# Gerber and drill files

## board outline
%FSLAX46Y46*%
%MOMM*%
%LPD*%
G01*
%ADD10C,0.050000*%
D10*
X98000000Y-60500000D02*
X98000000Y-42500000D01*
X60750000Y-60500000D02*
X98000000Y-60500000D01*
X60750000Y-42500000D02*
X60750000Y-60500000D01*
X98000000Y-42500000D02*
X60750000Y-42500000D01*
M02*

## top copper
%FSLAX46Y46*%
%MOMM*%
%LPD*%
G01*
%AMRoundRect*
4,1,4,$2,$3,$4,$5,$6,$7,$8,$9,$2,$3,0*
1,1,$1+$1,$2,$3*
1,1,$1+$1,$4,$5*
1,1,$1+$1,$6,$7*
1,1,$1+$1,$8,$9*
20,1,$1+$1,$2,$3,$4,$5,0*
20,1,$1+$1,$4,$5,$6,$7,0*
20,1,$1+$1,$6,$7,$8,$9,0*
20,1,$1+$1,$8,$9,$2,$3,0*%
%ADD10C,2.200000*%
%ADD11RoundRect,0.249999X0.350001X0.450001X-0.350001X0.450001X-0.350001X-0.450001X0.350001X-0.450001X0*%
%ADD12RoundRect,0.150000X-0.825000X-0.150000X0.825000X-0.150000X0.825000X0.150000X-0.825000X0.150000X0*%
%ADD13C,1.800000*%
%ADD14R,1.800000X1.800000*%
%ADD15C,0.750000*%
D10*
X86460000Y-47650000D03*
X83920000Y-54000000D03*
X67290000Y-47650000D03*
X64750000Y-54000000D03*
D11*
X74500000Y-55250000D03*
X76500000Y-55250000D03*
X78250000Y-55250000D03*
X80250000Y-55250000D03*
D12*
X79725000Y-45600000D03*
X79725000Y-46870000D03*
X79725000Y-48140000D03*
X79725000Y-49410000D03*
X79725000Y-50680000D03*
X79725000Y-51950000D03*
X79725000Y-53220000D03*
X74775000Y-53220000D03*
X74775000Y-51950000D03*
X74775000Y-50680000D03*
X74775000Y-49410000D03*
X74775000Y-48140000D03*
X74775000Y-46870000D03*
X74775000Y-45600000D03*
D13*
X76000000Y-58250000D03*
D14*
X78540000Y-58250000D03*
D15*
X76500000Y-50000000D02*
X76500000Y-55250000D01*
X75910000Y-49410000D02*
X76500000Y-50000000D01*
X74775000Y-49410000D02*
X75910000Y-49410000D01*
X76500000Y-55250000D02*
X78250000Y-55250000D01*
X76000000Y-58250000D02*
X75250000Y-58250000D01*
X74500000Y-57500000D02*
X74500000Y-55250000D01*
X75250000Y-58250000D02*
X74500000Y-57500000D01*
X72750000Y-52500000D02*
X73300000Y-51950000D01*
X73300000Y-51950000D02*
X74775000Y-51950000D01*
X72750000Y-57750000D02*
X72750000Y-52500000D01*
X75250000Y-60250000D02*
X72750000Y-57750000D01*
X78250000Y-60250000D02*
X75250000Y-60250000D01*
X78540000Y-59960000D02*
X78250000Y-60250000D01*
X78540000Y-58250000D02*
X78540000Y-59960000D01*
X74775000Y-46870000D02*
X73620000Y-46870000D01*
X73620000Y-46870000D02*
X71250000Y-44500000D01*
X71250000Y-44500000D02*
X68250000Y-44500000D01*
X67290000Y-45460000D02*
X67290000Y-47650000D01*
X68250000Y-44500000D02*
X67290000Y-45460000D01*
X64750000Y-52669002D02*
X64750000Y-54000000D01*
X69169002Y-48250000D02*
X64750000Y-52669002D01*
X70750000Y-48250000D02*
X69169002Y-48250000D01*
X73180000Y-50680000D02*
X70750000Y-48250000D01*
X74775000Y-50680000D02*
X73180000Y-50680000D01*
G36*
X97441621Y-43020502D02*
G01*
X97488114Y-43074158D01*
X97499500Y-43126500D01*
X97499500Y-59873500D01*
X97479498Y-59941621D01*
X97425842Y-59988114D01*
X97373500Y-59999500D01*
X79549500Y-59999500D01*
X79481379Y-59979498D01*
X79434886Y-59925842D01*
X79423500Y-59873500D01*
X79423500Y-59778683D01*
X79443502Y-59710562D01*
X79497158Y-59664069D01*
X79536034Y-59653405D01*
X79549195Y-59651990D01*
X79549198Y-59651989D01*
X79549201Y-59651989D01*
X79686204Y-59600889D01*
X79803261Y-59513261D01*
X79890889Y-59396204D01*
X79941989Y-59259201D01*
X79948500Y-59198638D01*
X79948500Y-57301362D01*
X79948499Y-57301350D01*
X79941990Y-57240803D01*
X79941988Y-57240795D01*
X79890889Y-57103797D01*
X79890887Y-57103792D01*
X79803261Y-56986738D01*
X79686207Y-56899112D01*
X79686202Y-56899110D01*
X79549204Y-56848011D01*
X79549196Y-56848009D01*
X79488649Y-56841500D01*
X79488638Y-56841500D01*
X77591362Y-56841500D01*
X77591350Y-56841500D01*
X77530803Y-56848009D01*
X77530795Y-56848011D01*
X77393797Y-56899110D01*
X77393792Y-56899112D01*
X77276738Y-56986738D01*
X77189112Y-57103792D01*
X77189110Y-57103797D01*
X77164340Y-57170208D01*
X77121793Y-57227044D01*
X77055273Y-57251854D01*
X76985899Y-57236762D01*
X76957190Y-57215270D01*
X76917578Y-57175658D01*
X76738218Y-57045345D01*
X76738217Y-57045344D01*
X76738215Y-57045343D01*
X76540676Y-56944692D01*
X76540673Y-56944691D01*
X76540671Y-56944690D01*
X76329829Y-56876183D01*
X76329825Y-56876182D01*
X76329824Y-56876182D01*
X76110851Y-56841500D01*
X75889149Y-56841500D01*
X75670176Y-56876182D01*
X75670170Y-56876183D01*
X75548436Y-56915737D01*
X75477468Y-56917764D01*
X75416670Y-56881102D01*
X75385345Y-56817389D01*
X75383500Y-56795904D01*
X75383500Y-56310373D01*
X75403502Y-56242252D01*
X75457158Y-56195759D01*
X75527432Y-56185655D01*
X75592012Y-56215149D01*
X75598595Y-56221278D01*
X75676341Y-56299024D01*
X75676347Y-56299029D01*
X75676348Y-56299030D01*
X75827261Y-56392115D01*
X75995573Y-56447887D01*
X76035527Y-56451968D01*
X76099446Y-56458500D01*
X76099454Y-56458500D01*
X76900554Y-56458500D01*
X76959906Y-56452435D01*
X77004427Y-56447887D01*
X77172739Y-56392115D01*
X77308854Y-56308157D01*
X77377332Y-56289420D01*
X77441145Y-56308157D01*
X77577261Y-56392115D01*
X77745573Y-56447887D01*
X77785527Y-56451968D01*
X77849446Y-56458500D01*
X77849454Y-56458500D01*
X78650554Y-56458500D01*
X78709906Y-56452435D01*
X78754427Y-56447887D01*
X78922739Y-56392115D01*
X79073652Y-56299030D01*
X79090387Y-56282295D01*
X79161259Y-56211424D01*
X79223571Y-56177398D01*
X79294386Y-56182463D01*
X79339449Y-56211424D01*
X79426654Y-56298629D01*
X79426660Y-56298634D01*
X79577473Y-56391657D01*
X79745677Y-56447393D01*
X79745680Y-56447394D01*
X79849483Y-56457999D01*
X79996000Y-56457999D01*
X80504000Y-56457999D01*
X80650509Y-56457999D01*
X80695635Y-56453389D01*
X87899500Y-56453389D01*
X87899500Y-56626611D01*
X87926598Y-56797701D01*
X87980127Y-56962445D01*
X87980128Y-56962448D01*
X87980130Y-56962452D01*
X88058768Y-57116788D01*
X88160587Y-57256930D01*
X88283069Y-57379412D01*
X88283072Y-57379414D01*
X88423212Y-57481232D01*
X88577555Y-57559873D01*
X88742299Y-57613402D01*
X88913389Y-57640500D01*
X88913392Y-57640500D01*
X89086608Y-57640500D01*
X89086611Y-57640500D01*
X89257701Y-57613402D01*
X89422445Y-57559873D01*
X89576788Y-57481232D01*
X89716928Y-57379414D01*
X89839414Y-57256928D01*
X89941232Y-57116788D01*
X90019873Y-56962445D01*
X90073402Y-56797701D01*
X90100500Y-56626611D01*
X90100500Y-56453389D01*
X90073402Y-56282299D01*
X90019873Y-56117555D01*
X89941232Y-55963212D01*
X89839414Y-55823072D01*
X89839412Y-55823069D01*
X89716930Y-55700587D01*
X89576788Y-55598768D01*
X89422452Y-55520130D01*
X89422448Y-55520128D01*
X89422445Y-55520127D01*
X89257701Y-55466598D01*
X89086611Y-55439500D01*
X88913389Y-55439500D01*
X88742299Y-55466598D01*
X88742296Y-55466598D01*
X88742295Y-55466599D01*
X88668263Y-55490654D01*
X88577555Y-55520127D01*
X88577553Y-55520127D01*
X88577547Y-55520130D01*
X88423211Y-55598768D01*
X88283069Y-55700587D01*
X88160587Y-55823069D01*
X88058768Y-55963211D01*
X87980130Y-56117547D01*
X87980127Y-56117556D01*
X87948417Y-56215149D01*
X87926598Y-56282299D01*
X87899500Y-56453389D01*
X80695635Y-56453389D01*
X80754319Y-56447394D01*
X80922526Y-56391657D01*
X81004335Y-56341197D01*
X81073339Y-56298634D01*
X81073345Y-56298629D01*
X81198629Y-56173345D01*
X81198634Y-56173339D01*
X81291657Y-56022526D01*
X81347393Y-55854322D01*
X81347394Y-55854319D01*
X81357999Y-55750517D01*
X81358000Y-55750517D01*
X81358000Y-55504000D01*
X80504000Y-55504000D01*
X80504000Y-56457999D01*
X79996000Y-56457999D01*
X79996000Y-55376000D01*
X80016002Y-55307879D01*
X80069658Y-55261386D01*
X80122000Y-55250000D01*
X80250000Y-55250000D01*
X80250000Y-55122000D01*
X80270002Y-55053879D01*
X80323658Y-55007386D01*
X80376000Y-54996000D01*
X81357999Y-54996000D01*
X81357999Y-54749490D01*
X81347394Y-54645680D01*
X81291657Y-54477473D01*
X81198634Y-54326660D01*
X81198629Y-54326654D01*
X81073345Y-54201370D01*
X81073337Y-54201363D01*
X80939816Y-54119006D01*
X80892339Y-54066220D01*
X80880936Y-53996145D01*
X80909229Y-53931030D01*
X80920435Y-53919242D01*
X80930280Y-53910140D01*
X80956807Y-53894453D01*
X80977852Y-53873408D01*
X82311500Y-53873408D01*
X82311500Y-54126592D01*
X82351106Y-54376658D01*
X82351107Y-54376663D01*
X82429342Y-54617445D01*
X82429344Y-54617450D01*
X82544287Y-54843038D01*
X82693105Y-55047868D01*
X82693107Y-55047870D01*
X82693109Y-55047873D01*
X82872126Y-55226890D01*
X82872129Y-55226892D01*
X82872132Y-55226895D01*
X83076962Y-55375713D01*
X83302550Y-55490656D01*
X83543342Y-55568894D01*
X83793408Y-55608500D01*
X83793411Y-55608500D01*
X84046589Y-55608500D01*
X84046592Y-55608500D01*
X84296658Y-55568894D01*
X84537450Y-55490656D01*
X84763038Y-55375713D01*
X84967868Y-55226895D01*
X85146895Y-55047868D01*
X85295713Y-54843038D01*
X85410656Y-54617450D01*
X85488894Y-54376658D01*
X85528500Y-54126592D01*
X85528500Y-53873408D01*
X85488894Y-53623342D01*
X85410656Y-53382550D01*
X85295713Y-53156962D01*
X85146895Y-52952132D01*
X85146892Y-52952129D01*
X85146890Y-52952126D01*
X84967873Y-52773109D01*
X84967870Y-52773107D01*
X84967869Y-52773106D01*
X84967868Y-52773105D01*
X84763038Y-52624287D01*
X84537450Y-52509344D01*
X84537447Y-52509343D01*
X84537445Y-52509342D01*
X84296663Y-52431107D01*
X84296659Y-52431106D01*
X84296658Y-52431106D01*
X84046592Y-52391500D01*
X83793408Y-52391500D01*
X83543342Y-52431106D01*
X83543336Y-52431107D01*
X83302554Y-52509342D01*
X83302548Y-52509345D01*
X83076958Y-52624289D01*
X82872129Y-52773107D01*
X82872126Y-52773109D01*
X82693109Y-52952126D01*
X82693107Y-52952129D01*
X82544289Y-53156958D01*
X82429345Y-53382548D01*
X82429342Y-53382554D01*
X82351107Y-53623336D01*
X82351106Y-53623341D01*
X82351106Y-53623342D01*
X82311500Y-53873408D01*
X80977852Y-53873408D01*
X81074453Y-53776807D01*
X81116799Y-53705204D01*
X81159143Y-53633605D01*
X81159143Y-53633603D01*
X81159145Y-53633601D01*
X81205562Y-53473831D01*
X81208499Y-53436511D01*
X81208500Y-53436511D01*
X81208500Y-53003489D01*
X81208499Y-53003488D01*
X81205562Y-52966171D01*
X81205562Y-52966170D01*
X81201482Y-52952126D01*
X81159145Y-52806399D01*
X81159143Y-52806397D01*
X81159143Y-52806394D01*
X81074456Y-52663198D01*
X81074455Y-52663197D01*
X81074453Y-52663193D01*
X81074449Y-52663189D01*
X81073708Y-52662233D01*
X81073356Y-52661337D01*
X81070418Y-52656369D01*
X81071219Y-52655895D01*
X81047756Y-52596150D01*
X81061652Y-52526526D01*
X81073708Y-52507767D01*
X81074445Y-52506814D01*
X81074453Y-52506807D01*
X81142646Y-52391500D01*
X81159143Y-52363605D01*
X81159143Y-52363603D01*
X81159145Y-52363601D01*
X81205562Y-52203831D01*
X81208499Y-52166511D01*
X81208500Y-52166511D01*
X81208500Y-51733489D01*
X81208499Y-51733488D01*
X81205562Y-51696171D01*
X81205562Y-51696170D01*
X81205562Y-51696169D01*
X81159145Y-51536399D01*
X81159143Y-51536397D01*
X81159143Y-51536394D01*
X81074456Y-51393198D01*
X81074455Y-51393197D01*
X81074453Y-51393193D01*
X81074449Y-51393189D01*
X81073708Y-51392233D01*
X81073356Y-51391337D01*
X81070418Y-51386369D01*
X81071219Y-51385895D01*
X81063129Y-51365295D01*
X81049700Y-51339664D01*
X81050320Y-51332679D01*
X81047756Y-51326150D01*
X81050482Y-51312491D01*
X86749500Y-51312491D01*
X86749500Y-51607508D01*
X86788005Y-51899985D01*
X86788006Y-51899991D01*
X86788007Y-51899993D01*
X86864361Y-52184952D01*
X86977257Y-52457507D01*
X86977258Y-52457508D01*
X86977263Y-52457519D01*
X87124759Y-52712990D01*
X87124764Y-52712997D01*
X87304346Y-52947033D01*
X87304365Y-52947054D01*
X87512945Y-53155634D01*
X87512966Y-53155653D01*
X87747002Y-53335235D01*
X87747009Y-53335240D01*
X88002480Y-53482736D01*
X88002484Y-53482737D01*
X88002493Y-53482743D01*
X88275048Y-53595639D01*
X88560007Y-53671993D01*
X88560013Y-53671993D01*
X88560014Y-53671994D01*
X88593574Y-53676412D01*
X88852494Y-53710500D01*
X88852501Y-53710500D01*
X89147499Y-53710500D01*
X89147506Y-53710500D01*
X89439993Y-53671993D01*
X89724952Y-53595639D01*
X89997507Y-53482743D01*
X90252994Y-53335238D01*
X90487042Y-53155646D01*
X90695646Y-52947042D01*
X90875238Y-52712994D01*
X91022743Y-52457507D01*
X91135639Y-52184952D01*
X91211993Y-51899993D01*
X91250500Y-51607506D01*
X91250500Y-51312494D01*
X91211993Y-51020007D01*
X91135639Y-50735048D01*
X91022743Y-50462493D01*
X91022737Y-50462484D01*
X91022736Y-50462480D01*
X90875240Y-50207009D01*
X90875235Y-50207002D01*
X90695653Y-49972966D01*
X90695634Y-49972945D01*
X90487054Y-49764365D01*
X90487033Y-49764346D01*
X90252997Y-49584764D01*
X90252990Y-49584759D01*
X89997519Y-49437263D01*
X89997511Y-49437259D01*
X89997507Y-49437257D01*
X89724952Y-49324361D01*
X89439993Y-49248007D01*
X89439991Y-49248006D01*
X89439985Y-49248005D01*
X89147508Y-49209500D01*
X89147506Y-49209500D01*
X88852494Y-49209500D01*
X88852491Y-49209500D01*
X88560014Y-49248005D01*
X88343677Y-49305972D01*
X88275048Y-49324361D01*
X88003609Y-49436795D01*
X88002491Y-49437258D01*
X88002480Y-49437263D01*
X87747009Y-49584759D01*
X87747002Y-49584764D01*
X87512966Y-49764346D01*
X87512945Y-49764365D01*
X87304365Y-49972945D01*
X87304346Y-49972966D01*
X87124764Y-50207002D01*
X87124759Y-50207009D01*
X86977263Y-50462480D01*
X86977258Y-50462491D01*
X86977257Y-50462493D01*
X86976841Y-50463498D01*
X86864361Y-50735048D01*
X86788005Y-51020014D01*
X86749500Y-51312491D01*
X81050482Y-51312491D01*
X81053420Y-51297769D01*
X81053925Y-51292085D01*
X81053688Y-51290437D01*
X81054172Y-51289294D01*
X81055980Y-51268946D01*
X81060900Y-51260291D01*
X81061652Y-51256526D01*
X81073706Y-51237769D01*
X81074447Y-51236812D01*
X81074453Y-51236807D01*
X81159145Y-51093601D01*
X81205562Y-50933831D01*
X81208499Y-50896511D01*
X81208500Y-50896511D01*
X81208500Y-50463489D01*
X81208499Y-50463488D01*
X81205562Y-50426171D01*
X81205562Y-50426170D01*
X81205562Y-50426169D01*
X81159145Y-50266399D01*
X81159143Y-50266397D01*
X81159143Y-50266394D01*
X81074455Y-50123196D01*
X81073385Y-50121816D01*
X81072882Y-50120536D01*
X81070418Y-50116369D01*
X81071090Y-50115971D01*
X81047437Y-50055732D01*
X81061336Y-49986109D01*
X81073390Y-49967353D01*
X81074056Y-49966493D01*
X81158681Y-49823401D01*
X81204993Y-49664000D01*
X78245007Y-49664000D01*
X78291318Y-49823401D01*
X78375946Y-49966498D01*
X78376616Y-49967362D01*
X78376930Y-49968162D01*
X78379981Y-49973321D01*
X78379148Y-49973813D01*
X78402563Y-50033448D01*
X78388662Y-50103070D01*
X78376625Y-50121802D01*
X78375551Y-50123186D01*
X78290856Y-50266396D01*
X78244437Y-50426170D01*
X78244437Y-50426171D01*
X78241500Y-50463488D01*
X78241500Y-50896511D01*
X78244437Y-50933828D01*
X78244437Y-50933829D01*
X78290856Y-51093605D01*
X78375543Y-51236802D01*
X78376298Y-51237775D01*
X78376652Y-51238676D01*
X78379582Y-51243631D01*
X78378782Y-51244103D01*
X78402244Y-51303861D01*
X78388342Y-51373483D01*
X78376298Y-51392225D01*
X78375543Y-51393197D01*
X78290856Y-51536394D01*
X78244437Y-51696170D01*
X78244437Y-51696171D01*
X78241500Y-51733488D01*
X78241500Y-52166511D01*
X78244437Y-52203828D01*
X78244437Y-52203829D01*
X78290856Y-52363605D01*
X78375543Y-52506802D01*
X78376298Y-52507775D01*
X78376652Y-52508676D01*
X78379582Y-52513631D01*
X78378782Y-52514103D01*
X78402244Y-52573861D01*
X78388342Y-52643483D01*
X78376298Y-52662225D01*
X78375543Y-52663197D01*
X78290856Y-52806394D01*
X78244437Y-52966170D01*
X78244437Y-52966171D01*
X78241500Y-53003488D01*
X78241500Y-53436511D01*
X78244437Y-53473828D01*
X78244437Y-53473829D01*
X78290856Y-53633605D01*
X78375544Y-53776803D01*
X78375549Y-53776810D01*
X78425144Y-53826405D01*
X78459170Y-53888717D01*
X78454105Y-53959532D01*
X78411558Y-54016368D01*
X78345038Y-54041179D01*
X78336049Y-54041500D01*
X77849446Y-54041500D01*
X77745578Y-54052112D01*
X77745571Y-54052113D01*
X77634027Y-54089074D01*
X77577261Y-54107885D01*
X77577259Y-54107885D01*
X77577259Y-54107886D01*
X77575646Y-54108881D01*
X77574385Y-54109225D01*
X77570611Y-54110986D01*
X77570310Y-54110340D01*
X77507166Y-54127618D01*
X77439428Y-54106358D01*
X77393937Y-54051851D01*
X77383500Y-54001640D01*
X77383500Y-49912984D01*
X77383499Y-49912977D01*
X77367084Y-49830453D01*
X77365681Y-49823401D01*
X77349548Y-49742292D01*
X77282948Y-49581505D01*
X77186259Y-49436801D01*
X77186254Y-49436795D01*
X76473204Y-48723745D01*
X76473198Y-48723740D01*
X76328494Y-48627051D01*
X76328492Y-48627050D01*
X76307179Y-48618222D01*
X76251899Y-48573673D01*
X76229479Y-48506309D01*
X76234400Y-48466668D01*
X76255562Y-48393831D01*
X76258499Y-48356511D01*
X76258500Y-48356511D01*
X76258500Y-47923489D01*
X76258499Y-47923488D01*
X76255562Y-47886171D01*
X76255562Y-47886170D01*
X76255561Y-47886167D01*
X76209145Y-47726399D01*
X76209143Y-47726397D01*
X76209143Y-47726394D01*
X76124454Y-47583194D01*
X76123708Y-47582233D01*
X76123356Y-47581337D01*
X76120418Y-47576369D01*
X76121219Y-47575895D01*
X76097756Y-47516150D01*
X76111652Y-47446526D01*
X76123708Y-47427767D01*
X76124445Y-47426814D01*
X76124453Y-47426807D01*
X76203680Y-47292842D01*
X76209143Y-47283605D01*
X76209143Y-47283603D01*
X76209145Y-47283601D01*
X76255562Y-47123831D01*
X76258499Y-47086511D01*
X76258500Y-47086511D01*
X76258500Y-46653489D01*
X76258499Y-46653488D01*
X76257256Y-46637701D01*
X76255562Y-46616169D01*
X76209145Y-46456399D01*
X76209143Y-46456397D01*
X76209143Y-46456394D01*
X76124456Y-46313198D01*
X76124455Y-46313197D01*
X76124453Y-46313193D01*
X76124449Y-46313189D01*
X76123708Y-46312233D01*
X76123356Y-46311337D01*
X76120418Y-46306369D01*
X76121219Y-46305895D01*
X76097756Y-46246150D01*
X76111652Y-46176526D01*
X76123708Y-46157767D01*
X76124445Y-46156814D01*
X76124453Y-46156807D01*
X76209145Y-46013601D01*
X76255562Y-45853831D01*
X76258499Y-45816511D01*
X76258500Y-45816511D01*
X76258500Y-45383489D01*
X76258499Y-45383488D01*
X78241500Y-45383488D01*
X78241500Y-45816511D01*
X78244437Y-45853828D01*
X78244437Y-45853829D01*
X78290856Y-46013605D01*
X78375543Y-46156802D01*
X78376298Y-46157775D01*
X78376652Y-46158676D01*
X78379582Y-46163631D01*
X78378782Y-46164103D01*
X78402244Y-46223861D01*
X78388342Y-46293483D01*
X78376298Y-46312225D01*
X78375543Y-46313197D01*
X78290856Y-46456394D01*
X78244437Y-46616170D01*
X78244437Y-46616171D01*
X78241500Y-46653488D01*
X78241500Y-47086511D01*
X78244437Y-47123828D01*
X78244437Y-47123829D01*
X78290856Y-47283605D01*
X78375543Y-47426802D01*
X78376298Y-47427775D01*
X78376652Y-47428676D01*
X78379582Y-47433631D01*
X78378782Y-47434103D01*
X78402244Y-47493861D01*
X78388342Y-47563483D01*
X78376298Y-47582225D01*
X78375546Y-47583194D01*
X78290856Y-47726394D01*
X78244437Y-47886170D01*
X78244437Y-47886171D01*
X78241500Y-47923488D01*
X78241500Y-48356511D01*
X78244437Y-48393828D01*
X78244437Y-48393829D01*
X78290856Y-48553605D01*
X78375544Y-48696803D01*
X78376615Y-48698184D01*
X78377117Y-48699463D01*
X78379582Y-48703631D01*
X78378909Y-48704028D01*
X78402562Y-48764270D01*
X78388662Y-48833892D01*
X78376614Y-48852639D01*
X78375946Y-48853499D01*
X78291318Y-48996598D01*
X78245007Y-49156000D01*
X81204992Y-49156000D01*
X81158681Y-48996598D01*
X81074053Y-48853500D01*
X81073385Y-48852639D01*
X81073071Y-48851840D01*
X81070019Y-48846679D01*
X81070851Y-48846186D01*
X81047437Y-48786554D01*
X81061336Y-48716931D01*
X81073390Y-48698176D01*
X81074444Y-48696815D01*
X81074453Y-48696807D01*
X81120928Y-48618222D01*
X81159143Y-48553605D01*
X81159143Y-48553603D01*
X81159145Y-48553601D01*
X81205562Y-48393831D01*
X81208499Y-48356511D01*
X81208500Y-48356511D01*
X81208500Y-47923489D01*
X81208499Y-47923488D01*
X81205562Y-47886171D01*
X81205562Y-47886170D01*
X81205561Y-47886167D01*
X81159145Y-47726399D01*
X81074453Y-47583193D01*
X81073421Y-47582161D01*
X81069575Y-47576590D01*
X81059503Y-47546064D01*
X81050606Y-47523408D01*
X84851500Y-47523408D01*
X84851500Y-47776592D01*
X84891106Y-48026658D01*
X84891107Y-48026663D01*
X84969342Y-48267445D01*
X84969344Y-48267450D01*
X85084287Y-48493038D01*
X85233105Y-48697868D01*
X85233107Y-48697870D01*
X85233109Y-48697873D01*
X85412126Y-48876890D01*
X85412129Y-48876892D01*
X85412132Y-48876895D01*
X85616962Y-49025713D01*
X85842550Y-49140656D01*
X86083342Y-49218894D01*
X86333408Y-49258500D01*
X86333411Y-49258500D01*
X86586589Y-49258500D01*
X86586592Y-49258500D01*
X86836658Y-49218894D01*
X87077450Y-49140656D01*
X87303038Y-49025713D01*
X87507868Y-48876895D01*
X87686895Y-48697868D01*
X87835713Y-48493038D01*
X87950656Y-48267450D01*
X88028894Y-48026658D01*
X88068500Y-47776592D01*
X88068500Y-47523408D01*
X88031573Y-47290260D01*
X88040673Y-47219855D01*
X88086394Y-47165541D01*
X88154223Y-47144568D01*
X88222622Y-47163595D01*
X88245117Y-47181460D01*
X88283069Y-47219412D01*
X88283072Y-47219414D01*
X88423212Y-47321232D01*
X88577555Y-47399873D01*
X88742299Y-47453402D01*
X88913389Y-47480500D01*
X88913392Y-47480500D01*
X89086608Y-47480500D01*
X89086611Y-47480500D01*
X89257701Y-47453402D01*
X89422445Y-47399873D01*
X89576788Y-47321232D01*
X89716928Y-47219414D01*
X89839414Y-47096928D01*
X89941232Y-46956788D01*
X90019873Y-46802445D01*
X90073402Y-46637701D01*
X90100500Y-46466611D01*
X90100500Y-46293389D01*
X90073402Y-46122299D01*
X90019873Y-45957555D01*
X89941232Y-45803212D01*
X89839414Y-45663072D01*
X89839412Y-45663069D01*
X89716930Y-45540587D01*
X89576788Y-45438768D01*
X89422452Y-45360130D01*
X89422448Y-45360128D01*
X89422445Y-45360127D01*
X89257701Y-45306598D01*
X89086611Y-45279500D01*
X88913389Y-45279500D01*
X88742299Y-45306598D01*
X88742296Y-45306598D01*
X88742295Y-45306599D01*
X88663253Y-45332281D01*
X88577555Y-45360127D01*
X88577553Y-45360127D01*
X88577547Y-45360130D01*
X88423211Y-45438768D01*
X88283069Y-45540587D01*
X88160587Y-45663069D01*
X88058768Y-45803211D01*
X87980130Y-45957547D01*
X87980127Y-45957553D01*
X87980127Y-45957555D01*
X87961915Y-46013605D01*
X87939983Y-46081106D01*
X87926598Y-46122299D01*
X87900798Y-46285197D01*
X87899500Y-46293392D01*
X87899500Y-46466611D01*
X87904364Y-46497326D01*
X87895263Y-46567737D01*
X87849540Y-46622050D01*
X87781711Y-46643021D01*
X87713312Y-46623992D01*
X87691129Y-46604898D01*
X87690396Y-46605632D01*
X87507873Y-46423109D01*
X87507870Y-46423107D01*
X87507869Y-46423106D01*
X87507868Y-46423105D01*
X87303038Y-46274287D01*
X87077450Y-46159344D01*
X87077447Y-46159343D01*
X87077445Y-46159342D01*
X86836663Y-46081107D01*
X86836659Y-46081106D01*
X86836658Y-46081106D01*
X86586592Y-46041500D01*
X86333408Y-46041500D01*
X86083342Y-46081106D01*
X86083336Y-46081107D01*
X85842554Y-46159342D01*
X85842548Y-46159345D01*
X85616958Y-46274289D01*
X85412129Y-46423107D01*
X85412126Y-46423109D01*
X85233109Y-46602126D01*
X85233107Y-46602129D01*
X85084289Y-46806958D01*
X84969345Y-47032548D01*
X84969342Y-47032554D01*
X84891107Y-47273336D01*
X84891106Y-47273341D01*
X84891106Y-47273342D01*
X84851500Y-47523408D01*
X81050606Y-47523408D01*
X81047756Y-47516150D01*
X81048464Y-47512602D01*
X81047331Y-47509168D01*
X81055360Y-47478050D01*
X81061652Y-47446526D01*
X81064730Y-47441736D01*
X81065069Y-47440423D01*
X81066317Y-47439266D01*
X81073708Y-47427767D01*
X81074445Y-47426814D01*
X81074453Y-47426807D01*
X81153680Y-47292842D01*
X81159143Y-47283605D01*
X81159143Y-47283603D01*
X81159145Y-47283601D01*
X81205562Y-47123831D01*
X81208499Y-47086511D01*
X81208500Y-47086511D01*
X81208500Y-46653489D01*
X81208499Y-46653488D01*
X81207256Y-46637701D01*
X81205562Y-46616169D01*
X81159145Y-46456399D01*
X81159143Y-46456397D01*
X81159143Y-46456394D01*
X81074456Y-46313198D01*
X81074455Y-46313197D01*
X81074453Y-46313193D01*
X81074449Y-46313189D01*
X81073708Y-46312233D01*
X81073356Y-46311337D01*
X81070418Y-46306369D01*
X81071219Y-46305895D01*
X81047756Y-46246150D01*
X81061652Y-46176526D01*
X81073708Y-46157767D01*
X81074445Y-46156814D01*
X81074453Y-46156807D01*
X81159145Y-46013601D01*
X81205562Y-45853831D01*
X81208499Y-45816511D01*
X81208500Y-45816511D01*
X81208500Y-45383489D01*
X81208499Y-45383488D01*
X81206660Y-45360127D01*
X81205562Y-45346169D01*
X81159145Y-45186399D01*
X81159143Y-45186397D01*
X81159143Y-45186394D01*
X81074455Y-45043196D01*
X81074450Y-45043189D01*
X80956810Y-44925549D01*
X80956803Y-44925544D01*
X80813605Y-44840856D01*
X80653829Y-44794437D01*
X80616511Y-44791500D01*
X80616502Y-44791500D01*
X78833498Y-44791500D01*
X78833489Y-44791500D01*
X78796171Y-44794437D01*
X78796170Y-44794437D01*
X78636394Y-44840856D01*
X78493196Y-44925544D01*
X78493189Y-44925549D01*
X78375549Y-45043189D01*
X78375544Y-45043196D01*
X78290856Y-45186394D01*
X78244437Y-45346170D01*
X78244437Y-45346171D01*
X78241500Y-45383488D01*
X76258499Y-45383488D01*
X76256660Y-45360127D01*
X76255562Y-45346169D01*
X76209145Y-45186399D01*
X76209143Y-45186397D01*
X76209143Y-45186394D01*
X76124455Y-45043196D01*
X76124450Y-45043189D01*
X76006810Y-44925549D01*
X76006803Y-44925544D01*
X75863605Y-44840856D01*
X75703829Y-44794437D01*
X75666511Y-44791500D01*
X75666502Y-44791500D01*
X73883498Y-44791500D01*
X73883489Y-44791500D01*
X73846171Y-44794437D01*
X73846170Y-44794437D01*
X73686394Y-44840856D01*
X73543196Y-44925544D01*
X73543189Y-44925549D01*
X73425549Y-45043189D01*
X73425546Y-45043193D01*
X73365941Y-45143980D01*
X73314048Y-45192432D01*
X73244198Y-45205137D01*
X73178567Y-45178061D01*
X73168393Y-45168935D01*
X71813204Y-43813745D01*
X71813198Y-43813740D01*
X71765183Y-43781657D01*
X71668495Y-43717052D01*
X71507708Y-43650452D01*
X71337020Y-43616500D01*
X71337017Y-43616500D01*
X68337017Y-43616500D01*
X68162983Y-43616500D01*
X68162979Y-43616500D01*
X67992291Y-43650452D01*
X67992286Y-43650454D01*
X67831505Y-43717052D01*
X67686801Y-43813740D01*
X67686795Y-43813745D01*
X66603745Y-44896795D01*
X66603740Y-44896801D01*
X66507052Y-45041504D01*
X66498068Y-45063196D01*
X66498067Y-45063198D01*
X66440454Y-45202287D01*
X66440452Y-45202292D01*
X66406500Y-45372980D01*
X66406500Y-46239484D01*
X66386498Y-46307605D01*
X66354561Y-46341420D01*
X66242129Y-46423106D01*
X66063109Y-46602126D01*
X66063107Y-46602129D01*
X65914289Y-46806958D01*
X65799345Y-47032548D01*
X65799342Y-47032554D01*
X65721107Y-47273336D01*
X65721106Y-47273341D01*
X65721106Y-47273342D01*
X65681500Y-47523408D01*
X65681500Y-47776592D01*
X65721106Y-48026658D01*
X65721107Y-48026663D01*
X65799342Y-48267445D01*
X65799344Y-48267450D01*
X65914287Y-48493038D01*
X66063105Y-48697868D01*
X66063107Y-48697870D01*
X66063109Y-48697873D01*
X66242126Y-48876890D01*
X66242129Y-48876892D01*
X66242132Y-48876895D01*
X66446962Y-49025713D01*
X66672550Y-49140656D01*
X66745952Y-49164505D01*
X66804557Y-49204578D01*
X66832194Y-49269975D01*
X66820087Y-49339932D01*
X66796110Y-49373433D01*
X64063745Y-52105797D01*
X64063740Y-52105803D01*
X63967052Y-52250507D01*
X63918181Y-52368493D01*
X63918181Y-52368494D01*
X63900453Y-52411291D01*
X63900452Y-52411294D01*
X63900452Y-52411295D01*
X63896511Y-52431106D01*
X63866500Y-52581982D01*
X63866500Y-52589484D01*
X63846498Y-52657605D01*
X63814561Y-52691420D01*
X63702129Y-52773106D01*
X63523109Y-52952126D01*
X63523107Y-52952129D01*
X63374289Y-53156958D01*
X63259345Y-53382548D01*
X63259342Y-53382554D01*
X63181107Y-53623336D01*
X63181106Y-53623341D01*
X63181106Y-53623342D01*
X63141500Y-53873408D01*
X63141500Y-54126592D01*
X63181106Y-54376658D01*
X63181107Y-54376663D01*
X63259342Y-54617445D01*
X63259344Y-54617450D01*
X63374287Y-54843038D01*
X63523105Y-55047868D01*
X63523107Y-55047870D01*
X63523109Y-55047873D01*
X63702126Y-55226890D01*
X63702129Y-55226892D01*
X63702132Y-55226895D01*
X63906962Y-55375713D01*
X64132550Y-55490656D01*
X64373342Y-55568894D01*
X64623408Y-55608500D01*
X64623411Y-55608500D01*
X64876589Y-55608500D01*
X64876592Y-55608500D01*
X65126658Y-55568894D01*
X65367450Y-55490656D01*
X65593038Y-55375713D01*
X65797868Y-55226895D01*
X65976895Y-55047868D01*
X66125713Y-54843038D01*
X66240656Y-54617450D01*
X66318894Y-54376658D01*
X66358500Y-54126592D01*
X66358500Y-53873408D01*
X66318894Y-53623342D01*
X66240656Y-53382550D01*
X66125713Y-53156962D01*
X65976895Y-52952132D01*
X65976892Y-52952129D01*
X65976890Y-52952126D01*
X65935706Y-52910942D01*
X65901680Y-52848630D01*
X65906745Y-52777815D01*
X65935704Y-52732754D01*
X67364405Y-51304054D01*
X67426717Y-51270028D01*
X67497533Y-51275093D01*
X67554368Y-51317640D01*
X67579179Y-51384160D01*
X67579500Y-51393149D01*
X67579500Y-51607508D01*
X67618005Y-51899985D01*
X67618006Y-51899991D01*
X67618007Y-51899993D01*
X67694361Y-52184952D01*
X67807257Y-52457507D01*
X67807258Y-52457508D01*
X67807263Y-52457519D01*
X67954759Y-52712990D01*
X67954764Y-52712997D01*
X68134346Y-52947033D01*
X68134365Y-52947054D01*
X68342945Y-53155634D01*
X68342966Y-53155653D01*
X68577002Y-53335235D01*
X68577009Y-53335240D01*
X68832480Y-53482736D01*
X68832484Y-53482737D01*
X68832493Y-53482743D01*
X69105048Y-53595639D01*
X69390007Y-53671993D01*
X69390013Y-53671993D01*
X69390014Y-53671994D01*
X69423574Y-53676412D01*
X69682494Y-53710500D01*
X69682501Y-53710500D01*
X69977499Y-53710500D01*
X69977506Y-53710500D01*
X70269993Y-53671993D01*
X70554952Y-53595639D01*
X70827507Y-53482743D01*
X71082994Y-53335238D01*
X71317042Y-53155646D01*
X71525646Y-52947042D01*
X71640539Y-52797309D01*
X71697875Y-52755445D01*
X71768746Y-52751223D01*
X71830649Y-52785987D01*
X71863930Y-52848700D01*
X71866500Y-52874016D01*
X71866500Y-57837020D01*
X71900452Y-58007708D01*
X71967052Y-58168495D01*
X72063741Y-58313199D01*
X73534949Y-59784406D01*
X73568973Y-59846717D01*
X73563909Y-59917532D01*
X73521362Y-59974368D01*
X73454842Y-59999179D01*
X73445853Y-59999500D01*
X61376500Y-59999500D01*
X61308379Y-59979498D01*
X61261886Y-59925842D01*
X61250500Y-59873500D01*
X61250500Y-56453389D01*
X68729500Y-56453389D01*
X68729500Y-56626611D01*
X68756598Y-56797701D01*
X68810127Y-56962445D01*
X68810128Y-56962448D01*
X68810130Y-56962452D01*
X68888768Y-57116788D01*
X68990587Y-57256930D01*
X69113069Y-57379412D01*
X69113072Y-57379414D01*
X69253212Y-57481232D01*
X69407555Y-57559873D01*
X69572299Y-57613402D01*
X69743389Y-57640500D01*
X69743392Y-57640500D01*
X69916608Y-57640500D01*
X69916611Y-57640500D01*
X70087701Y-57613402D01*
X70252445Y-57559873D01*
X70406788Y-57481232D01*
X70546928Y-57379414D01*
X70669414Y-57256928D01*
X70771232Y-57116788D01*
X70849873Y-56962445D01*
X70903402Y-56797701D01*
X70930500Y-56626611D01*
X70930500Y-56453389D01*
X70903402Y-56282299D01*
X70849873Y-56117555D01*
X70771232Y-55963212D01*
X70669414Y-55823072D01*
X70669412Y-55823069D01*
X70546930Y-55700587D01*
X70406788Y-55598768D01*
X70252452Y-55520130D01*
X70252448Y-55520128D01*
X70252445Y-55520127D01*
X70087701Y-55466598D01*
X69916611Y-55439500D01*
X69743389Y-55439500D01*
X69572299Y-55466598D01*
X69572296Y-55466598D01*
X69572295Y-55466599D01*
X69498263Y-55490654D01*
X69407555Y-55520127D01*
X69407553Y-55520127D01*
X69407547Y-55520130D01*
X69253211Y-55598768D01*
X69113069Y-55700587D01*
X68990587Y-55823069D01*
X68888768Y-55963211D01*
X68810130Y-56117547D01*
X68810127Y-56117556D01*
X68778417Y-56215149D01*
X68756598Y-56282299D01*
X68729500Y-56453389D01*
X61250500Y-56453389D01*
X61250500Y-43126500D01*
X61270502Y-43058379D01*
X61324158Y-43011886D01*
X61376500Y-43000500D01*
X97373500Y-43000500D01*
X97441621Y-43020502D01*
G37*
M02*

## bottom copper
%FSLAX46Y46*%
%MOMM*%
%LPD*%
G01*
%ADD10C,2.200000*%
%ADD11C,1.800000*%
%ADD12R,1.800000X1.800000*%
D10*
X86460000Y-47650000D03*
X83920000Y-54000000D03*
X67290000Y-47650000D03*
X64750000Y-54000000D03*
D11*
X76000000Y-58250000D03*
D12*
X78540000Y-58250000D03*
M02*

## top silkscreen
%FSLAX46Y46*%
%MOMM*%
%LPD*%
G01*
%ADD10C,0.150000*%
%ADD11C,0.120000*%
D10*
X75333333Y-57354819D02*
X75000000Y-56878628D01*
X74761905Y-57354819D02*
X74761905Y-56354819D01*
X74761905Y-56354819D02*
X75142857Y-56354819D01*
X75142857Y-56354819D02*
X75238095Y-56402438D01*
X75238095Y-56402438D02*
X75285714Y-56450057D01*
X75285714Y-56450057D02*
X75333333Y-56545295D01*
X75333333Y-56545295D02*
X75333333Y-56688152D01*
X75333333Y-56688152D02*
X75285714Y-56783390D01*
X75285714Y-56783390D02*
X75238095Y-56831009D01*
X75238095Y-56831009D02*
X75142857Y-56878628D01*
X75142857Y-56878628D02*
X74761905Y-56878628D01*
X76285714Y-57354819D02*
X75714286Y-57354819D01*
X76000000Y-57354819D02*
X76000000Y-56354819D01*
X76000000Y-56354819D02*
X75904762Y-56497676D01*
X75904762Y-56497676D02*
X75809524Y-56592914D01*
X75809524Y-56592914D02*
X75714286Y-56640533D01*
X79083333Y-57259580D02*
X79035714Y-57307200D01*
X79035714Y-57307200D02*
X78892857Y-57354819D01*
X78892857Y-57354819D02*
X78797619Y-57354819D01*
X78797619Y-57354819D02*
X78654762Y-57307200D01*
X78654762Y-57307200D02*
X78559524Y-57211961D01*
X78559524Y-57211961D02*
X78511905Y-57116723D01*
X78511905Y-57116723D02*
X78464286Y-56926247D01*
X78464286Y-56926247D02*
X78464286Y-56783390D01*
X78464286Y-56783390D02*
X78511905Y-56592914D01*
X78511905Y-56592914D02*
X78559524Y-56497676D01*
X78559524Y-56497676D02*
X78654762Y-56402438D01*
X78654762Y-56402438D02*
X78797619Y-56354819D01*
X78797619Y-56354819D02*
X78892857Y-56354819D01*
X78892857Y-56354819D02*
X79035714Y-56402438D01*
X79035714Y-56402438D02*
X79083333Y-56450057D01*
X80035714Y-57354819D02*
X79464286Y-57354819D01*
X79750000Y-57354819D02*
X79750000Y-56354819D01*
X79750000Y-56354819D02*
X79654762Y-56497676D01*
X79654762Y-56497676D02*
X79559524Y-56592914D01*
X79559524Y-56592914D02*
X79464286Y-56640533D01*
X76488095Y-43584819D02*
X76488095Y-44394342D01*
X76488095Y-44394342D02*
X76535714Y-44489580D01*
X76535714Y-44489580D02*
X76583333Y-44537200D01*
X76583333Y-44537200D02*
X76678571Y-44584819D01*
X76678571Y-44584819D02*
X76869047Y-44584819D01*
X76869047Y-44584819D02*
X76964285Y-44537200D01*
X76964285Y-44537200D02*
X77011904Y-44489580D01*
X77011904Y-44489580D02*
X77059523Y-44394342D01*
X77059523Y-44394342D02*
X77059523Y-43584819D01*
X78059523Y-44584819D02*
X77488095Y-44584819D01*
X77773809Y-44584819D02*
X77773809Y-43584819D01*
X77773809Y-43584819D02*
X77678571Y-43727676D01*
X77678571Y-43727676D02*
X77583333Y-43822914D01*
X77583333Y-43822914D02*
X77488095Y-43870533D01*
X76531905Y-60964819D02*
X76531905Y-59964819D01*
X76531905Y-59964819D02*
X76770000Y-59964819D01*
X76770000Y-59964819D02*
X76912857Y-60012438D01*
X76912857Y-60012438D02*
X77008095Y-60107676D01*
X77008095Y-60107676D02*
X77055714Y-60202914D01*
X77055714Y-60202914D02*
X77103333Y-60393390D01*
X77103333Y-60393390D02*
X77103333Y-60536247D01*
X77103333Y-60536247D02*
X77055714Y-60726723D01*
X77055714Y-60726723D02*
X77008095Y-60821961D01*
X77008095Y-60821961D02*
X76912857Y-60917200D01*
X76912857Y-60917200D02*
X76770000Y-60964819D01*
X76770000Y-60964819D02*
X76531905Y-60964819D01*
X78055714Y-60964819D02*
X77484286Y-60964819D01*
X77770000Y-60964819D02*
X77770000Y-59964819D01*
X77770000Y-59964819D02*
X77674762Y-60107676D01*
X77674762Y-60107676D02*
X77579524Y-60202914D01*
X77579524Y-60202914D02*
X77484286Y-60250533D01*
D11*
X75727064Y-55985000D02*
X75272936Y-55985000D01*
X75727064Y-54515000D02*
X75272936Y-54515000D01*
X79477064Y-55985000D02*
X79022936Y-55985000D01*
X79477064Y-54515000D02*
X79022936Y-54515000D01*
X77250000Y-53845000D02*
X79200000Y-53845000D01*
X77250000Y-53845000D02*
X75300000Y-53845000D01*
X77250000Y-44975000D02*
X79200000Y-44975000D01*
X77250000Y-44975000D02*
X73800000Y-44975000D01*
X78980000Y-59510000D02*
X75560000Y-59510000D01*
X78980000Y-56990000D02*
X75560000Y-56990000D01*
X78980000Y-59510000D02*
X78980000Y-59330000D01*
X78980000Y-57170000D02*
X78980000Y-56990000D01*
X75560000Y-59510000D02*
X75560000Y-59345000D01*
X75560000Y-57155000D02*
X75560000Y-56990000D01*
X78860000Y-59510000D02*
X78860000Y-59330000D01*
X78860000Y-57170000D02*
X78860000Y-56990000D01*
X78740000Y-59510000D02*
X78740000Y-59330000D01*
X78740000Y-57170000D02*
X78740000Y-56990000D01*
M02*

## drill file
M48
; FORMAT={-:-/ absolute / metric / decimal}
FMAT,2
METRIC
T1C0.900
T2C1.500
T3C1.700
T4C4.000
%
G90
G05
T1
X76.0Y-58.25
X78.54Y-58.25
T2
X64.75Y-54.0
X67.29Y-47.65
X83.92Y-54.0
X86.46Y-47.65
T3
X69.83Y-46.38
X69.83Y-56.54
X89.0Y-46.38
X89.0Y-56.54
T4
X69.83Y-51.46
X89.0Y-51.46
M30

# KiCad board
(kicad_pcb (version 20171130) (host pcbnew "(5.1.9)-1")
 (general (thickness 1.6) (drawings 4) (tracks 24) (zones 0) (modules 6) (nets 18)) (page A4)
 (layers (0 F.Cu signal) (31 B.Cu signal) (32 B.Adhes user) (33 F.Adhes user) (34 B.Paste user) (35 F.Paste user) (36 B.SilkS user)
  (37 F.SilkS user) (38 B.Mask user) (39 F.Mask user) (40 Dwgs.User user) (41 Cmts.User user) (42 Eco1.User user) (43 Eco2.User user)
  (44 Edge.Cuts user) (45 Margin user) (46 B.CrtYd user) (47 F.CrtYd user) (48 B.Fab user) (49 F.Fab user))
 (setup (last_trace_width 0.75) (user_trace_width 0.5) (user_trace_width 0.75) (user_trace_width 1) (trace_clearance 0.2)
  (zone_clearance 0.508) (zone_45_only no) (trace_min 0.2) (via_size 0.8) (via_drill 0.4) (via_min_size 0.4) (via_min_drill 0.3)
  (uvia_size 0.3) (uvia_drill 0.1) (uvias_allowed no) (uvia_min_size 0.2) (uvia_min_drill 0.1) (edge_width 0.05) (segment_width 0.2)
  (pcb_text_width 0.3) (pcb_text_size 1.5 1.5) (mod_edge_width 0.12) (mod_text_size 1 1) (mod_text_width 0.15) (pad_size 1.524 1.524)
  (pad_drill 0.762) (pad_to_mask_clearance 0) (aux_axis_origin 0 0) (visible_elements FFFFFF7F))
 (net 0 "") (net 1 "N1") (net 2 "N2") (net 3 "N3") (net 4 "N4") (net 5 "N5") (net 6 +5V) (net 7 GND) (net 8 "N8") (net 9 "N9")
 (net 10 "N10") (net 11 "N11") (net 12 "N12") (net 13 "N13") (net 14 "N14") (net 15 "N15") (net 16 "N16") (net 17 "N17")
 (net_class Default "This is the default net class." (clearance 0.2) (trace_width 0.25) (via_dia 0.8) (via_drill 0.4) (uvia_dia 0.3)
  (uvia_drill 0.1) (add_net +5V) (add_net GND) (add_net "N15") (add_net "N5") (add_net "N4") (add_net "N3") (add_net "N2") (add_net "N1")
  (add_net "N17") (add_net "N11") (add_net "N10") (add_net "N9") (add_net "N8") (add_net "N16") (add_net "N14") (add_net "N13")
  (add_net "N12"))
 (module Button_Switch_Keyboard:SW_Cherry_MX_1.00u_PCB (layer B.Cu) (at 83.92 54 270)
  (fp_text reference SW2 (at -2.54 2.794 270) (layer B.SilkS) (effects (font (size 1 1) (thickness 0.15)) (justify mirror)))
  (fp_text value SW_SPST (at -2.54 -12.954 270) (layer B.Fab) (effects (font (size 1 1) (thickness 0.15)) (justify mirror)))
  (pad "" np_thru_hole circle (at 2.54 -5.08 270) (size 1.7 1.7) (drill 1.7) (layers *.Cu *.Mask))
  (pad "" np_thru_hole circle (at -7.62 -5.08 270) (size 1.7 1.7) (drill 1.7) (layers *.Cu *.Mask))
  (pad "" np_thru_hole circle (at -2.54 -5.08 270) (size 4 4) (drill 4) (layers *.Cu *.Mask))
  (pad 2 thru_hole circle (at -6.35 -2.54 270) (size 2.2 2.2) (drill 1.5) (layers *.Cu *.Mask) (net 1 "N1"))
  (pad 1 thru_hole circle (at 0 0 270) (size 2.2 2.2) (drill 1.5) (layers *.Cu *.Mask) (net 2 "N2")))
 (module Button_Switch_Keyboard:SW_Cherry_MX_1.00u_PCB (layer B.Cu) (at 64.75 54 270)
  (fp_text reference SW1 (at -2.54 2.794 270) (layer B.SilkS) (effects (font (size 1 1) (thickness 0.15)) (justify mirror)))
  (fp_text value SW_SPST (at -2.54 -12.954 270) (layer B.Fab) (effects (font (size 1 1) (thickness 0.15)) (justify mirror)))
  (pad "" np_thru_hole circle (at 2.54 -5.08 270) (size 1.7 1.7) (drill 1.7) (layers *.Cu *.Mask))
  (pad "" np_thru_hole circle (at -7.62 -5.08 270) (size 1.7 1.7) (drill 1.7) (layers *.Cu *.Mask))
  (pad "" np_thru_hole circle (at -2.54 -5.08 270) (size 4 4) (drill 4) (layers *.Cu *.Mask))
  (pad 2 thru_hole circle (at -6.35 -2.54 270) (size 2.2 2.2) (drill 1.5) (layers *.Cu *.Mask) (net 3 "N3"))
  (pad 1 thru_hole circle (at 0 0 270) (size 2.2 2.2) (drill 1.5) (layers *.Cu *.Mask) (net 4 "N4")))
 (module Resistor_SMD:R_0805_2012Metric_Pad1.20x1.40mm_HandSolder (layer F.Cu) (at 75.5 55.25 180)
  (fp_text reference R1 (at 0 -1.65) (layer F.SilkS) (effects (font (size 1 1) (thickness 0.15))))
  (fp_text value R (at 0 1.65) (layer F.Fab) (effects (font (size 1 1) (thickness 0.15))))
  (fp_line (start -0.227064 -0.735) (end 0.227064 -0.735) (layer F.SilkS) (width 0.12))
  (fp_line (start -0.227064 0.735) (end 0.227064 0.735) (layer F.SilkS) (width 0.12))
  (pad 2 smd roundrect (at 1 0 180) (size 1.2 1.4) (layers F.Cu F.Paste F.Mask) (roundrect_rratio 0.2083325) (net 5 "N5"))
  (pad 1 smd roundrect (at -1 0 180) (size 1.2 1.4) (layers F.Cu F.Paste F.Mask) (roundrect_rratio 0.2083325) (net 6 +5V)))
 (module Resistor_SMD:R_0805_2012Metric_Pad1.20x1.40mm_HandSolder (layer F.Cu) (at 79.25 55.25 180)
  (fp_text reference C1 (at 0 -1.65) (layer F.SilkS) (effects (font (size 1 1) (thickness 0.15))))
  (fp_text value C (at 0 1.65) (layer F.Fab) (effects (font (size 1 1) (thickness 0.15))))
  (fp_line (start -0.227064 -0.735) (end 0.227064 -0.735) (layer F.SilkS) (width 0.12))
  (fp_line (start -0.227064 0.735) (end 0.227064 0.735) (layer F.SilkS) (width 0.12))
  (pad 2 smd roundrect (at 1 0 180) (size 1.2 1.4) (layers F.Cu F.Paste F.Mask) (roundrect_rratio 0.2083325) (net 6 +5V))
  (pad 1 smd roundrect (at -1 0 180) (size 1.2 1.4) (layers F.Cu F.Paste F.Mask) (roundrect_rratio 0.2083325) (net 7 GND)))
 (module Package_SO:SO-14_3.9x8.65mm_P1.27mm (layer F.Cu) (at 77.25 49.41)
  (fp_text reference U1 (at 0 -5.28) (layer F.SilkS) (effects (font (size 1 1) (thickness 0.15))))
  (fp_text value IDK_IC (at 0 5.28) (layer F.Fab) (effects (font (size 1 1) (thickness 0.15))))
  (fp_line (start 0 4.435) (end 1.95 4.435) (layer F.SilkS) (width 0.12))
  (fp_line (start 0 4.435) (end -1.95 4.435) (layer F.SilkS) (width 0.12))
  (fp_line (start 0 -4.435) (end 1.95 -4.435) (layer F.SilkS) (width 0.12))
  (fp_line (start 0 -4.435) (end -3.45 -4.435) (layer F.SilkS) (width 0.12))
  (pad 14 smd roundrect (at 2.475 -3.81) (size 1.95 0.6) (layers F.Cu F.Paste F.Mask) (roundrect_rratio 0.25) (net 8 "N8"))
  (pad 13 smd roundrect (at 2.475 -2.54) (size 1.95 0.6) (layers F.Cu F.Paste F.Mask) (roundrect_rratio 0.25) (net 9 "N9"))
  (pad 12 smd roundrect (at 2.475 -1.27) (size 1.95 0.6) (layers F.Cu F.Paste F.Mask) (roundrect_rratio 0.25) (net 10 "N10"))
  (pad 11 smd roundrect (at 2.475 0) (size 1.95 0.6) (layers F.Cu F.Paste F.Mask) (roundrect_rratio 0.25) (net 7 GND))
  (pad 10 smd roundrect (at 2.475 1.27) (size 1.95 0.6) (layers F.Cu F.Paste F.Mask) (roundrect_rratio 0.25) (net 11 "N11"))
  (pad 9 smd roundrect (at 2.475 2.54) (size 1.95 0.6) (layers F.Cu F.Paste F.Mask) (roundrect_rratio 0.25) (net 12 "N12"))
  (pad 8 smd roundrect (at 2.475 3.81) (size 1.95 0.6) (layers F.Cu F.Paste F.Mask) (roundrect_rratio 0.25) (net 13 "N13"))
  (pad 7 smd roundrect (at -2.475 3.81) (size 1.95 0.6) (layers F.Cu F.Paste F.Mask) (roundrect_rratio 0.25) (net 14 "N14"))
  (pad 6 smd roundrect (at -2.475 2.54) (size 1.95 0.6) (layers F.Cu F.Paste F.Mask) (roundrect_rratio 0.25) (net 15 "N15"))
  (pad 5 smd roundrect (at -2.475 1.27) (size 1.95 0.6) (layers F.Cu F.Paste F.Mask) (roundrect_rratio 0.25) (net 4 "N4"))
  (pad 4 smd roundrect (at -2.475 0) (size 1.95 0.6) (layers F.Cu F.Paste F.Mask) (roundrect_rratio 0.25) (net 6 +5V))
  (pad 3 smd roundrect (at -2.475 -1.27) (size 1.95 0.6) (layers F.Cu F.Paste F.Mask) (roundrect_rratio 0.25) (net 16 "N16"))
  (pad 2 smd roundrect (at -2.475 -2.54) (size 1.95 0.6) (layers F.Cu F.Paste F.Mask) (roundrect_rratio 0.25) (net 3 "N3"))
  (pad 1 smd roundrect (at -2.475 -3.81) (size 1.95 0.6) (layers F.Cu F.Paste F.Mask) (roundrect_rratio 0.25) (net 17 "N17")))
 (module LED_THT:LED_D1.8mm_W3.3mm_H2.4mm (layer F.Cu) (at 78.54 58.25 180)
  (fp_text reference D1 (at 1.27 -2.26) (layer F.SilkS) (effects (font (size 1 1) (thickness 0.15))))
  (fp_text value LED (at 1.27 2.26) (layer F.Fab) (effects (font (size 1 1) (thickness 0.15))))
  (fp_line (start -0.44 -1.26) (end 2.98 -1.26) (layer F.SilkS) (width 0.12))
  (fp_line (start -0.44 1.26) (end 2.98 1.26) (layer F.SilkS) (width 0.12))
  (fp_line (start -0.44 -1.26) (end -0.44 -1.08) (layer F.SilkS) (width 0.12))
  (fp_line (start -0.44 1.08) (end -0.44 1.26) (layer F.SilkS) (width 0.12))
  (fp_line (start 2.98 -1.26) (end 2.98 -1.095) (layer F.SilkS) (width 0.12))
  (fp_line (start 2.98 1.095) (end 2.98 1.26) (layer F.SilkS) (width 0.12))
  (fp_line (start -0.32 -1.26) (end -0.32 -1.08) (layer F.SilkS) (width 0.12))
  (fp_line (start -0.32 1.08) (end -0.32 1.26) (layer F.SilkS) (width 0.12))
  (fp_line (start -0.2 -1.26) (end -0.2 -1.08) (layer F.SilkS) (width 0.12))
  (fp_line (start -0.2 1.08) (end -0.2 1.26) (layer F.SilkS) (width 0.12))
  (pad 2 thru_hole circle (at 2.54 0 180) (size 1.8 1.8) (drill 0.9) (layers *.Cu *.Mask) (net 5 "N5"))
  (pad 1 thru_hole rect (at 0 0 180) (size 1.8 1.8) (drill 0.9) (layers *.Cu *.Mask) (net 15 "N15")))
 (gr_line (start 98 60.5) (end 98 42.5) (layer Edge.Cuts) (width 0.05))
 (gr_line (start 60.75 60.5) (end 98 60.5) (layer Edge.Cuts) (width 0.05))
 (gr_line (start 60.75 42.5) (end 60.75 60.5) (layer Edge.Cuts) (width 0.05))
 (gr_line (start 98 42.5) (end 60.75 42.5) (layer Edge.Cuts) (width 0.05))
 (segment (start 76.5 50) (end 76.5 55.25) (width 0.75) (layer F.Cu) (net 6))
 (segment (start 75.91 49.41) (end 76.5 50) (width 0.75) (layer F.Cu) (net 6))
 (segment (start 74.775 49.41) (end 75.91 49.41) (width 0.75) (layer F.Cu) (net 6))
 (segment (start 76.5 55.25) (end 78.25 55.25) (width 0.75) (layer F.Cu) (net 6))
 (segment (start 76 58.25) (end 75.25 58.25) (width 0.75) (layer F.Cu) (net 5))
 (segment (start 74.5 57.5) (end 74.5 55.25) (width 0.75) (layer F.Cu) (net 5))
 (segment (start 75.25 58.25) (end 74.5 57.5) (width 0.75) (layer F.Cu) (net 5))
 (segment (start 72.75 52.5) (end 73.3 51.95) (width 0.75) (layer F.Cu) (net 15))
 (segment (start 73.3 51.95) (end 74.775 51.95) (width 0.75) (layer F.Cu) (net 15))
 (segment (start 72.75 57.75) (end 72.75 52.5) (width 0.75) (layer F.Cu) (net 15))
 (segment (start 75.25 60.25) (end 72.75 57.75) (width 0.75) (layer F.Cu) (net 15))
 (segment (start 78.25 60.25) (end 75.25 60.25) (width 0.75) (layer F.Cu) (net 15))
 (segment (start 78.54 59.96) (end 78.25 60.25) (width 0.75) (layer F.Cu) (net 15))
 (segment (start 78.54 58.25) (end 78.54 59.96) (width 0.75) (layer F.Cu) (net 15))
 (segment (start 74.775 46.87) (end 73.62 46.87) (width 0.75) (layer F.Cu) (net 3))
 (segment (start 73.62 46.87) (end 71.25 44.5) (width 0.75) (layer F.Cu) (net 3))
 (segment (start 71.25 44.5) (end 68.25 44.5) (width 0.75) (layer F.Cu) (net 3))
 (segment (start 67.29 45.46) (end 67.29 47.65) (width 0.75) (layer F.Cu) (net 3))
 (segment (start 68.25 44.5) (end 67.29 45.46) (width 0.75) (layer F.Cu) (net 3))
 (segment (start 64.75 52.669002) (end 64.75 54) (width 0.75) (layer F.Cu) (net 4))
 (segment (start 69.169002 48.25) (end 64.75 52.669002) (width 0.75) (layer F.Cu) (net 4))
 (segment (start 70.75 48.25) (end 69.169002 48.25) (width 0.75) (layer F.Cu) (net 4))
 (segment (start 73.18 50.68) (end 70.75 48.25) (width 0.75) (layer F.Cu) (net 4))
 (segment (start 74.775 50.68) (end 73.18 50.68) (width 0.75) (layer F.Cu) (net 4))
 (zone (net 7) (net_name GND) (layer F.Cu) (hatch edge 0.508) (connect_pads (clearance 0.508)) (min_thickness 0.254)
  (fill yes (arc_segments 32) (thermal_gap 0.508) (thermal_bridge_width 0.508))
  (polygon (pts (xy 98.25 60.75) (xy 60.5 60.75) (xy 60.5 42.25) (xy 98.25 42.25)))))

